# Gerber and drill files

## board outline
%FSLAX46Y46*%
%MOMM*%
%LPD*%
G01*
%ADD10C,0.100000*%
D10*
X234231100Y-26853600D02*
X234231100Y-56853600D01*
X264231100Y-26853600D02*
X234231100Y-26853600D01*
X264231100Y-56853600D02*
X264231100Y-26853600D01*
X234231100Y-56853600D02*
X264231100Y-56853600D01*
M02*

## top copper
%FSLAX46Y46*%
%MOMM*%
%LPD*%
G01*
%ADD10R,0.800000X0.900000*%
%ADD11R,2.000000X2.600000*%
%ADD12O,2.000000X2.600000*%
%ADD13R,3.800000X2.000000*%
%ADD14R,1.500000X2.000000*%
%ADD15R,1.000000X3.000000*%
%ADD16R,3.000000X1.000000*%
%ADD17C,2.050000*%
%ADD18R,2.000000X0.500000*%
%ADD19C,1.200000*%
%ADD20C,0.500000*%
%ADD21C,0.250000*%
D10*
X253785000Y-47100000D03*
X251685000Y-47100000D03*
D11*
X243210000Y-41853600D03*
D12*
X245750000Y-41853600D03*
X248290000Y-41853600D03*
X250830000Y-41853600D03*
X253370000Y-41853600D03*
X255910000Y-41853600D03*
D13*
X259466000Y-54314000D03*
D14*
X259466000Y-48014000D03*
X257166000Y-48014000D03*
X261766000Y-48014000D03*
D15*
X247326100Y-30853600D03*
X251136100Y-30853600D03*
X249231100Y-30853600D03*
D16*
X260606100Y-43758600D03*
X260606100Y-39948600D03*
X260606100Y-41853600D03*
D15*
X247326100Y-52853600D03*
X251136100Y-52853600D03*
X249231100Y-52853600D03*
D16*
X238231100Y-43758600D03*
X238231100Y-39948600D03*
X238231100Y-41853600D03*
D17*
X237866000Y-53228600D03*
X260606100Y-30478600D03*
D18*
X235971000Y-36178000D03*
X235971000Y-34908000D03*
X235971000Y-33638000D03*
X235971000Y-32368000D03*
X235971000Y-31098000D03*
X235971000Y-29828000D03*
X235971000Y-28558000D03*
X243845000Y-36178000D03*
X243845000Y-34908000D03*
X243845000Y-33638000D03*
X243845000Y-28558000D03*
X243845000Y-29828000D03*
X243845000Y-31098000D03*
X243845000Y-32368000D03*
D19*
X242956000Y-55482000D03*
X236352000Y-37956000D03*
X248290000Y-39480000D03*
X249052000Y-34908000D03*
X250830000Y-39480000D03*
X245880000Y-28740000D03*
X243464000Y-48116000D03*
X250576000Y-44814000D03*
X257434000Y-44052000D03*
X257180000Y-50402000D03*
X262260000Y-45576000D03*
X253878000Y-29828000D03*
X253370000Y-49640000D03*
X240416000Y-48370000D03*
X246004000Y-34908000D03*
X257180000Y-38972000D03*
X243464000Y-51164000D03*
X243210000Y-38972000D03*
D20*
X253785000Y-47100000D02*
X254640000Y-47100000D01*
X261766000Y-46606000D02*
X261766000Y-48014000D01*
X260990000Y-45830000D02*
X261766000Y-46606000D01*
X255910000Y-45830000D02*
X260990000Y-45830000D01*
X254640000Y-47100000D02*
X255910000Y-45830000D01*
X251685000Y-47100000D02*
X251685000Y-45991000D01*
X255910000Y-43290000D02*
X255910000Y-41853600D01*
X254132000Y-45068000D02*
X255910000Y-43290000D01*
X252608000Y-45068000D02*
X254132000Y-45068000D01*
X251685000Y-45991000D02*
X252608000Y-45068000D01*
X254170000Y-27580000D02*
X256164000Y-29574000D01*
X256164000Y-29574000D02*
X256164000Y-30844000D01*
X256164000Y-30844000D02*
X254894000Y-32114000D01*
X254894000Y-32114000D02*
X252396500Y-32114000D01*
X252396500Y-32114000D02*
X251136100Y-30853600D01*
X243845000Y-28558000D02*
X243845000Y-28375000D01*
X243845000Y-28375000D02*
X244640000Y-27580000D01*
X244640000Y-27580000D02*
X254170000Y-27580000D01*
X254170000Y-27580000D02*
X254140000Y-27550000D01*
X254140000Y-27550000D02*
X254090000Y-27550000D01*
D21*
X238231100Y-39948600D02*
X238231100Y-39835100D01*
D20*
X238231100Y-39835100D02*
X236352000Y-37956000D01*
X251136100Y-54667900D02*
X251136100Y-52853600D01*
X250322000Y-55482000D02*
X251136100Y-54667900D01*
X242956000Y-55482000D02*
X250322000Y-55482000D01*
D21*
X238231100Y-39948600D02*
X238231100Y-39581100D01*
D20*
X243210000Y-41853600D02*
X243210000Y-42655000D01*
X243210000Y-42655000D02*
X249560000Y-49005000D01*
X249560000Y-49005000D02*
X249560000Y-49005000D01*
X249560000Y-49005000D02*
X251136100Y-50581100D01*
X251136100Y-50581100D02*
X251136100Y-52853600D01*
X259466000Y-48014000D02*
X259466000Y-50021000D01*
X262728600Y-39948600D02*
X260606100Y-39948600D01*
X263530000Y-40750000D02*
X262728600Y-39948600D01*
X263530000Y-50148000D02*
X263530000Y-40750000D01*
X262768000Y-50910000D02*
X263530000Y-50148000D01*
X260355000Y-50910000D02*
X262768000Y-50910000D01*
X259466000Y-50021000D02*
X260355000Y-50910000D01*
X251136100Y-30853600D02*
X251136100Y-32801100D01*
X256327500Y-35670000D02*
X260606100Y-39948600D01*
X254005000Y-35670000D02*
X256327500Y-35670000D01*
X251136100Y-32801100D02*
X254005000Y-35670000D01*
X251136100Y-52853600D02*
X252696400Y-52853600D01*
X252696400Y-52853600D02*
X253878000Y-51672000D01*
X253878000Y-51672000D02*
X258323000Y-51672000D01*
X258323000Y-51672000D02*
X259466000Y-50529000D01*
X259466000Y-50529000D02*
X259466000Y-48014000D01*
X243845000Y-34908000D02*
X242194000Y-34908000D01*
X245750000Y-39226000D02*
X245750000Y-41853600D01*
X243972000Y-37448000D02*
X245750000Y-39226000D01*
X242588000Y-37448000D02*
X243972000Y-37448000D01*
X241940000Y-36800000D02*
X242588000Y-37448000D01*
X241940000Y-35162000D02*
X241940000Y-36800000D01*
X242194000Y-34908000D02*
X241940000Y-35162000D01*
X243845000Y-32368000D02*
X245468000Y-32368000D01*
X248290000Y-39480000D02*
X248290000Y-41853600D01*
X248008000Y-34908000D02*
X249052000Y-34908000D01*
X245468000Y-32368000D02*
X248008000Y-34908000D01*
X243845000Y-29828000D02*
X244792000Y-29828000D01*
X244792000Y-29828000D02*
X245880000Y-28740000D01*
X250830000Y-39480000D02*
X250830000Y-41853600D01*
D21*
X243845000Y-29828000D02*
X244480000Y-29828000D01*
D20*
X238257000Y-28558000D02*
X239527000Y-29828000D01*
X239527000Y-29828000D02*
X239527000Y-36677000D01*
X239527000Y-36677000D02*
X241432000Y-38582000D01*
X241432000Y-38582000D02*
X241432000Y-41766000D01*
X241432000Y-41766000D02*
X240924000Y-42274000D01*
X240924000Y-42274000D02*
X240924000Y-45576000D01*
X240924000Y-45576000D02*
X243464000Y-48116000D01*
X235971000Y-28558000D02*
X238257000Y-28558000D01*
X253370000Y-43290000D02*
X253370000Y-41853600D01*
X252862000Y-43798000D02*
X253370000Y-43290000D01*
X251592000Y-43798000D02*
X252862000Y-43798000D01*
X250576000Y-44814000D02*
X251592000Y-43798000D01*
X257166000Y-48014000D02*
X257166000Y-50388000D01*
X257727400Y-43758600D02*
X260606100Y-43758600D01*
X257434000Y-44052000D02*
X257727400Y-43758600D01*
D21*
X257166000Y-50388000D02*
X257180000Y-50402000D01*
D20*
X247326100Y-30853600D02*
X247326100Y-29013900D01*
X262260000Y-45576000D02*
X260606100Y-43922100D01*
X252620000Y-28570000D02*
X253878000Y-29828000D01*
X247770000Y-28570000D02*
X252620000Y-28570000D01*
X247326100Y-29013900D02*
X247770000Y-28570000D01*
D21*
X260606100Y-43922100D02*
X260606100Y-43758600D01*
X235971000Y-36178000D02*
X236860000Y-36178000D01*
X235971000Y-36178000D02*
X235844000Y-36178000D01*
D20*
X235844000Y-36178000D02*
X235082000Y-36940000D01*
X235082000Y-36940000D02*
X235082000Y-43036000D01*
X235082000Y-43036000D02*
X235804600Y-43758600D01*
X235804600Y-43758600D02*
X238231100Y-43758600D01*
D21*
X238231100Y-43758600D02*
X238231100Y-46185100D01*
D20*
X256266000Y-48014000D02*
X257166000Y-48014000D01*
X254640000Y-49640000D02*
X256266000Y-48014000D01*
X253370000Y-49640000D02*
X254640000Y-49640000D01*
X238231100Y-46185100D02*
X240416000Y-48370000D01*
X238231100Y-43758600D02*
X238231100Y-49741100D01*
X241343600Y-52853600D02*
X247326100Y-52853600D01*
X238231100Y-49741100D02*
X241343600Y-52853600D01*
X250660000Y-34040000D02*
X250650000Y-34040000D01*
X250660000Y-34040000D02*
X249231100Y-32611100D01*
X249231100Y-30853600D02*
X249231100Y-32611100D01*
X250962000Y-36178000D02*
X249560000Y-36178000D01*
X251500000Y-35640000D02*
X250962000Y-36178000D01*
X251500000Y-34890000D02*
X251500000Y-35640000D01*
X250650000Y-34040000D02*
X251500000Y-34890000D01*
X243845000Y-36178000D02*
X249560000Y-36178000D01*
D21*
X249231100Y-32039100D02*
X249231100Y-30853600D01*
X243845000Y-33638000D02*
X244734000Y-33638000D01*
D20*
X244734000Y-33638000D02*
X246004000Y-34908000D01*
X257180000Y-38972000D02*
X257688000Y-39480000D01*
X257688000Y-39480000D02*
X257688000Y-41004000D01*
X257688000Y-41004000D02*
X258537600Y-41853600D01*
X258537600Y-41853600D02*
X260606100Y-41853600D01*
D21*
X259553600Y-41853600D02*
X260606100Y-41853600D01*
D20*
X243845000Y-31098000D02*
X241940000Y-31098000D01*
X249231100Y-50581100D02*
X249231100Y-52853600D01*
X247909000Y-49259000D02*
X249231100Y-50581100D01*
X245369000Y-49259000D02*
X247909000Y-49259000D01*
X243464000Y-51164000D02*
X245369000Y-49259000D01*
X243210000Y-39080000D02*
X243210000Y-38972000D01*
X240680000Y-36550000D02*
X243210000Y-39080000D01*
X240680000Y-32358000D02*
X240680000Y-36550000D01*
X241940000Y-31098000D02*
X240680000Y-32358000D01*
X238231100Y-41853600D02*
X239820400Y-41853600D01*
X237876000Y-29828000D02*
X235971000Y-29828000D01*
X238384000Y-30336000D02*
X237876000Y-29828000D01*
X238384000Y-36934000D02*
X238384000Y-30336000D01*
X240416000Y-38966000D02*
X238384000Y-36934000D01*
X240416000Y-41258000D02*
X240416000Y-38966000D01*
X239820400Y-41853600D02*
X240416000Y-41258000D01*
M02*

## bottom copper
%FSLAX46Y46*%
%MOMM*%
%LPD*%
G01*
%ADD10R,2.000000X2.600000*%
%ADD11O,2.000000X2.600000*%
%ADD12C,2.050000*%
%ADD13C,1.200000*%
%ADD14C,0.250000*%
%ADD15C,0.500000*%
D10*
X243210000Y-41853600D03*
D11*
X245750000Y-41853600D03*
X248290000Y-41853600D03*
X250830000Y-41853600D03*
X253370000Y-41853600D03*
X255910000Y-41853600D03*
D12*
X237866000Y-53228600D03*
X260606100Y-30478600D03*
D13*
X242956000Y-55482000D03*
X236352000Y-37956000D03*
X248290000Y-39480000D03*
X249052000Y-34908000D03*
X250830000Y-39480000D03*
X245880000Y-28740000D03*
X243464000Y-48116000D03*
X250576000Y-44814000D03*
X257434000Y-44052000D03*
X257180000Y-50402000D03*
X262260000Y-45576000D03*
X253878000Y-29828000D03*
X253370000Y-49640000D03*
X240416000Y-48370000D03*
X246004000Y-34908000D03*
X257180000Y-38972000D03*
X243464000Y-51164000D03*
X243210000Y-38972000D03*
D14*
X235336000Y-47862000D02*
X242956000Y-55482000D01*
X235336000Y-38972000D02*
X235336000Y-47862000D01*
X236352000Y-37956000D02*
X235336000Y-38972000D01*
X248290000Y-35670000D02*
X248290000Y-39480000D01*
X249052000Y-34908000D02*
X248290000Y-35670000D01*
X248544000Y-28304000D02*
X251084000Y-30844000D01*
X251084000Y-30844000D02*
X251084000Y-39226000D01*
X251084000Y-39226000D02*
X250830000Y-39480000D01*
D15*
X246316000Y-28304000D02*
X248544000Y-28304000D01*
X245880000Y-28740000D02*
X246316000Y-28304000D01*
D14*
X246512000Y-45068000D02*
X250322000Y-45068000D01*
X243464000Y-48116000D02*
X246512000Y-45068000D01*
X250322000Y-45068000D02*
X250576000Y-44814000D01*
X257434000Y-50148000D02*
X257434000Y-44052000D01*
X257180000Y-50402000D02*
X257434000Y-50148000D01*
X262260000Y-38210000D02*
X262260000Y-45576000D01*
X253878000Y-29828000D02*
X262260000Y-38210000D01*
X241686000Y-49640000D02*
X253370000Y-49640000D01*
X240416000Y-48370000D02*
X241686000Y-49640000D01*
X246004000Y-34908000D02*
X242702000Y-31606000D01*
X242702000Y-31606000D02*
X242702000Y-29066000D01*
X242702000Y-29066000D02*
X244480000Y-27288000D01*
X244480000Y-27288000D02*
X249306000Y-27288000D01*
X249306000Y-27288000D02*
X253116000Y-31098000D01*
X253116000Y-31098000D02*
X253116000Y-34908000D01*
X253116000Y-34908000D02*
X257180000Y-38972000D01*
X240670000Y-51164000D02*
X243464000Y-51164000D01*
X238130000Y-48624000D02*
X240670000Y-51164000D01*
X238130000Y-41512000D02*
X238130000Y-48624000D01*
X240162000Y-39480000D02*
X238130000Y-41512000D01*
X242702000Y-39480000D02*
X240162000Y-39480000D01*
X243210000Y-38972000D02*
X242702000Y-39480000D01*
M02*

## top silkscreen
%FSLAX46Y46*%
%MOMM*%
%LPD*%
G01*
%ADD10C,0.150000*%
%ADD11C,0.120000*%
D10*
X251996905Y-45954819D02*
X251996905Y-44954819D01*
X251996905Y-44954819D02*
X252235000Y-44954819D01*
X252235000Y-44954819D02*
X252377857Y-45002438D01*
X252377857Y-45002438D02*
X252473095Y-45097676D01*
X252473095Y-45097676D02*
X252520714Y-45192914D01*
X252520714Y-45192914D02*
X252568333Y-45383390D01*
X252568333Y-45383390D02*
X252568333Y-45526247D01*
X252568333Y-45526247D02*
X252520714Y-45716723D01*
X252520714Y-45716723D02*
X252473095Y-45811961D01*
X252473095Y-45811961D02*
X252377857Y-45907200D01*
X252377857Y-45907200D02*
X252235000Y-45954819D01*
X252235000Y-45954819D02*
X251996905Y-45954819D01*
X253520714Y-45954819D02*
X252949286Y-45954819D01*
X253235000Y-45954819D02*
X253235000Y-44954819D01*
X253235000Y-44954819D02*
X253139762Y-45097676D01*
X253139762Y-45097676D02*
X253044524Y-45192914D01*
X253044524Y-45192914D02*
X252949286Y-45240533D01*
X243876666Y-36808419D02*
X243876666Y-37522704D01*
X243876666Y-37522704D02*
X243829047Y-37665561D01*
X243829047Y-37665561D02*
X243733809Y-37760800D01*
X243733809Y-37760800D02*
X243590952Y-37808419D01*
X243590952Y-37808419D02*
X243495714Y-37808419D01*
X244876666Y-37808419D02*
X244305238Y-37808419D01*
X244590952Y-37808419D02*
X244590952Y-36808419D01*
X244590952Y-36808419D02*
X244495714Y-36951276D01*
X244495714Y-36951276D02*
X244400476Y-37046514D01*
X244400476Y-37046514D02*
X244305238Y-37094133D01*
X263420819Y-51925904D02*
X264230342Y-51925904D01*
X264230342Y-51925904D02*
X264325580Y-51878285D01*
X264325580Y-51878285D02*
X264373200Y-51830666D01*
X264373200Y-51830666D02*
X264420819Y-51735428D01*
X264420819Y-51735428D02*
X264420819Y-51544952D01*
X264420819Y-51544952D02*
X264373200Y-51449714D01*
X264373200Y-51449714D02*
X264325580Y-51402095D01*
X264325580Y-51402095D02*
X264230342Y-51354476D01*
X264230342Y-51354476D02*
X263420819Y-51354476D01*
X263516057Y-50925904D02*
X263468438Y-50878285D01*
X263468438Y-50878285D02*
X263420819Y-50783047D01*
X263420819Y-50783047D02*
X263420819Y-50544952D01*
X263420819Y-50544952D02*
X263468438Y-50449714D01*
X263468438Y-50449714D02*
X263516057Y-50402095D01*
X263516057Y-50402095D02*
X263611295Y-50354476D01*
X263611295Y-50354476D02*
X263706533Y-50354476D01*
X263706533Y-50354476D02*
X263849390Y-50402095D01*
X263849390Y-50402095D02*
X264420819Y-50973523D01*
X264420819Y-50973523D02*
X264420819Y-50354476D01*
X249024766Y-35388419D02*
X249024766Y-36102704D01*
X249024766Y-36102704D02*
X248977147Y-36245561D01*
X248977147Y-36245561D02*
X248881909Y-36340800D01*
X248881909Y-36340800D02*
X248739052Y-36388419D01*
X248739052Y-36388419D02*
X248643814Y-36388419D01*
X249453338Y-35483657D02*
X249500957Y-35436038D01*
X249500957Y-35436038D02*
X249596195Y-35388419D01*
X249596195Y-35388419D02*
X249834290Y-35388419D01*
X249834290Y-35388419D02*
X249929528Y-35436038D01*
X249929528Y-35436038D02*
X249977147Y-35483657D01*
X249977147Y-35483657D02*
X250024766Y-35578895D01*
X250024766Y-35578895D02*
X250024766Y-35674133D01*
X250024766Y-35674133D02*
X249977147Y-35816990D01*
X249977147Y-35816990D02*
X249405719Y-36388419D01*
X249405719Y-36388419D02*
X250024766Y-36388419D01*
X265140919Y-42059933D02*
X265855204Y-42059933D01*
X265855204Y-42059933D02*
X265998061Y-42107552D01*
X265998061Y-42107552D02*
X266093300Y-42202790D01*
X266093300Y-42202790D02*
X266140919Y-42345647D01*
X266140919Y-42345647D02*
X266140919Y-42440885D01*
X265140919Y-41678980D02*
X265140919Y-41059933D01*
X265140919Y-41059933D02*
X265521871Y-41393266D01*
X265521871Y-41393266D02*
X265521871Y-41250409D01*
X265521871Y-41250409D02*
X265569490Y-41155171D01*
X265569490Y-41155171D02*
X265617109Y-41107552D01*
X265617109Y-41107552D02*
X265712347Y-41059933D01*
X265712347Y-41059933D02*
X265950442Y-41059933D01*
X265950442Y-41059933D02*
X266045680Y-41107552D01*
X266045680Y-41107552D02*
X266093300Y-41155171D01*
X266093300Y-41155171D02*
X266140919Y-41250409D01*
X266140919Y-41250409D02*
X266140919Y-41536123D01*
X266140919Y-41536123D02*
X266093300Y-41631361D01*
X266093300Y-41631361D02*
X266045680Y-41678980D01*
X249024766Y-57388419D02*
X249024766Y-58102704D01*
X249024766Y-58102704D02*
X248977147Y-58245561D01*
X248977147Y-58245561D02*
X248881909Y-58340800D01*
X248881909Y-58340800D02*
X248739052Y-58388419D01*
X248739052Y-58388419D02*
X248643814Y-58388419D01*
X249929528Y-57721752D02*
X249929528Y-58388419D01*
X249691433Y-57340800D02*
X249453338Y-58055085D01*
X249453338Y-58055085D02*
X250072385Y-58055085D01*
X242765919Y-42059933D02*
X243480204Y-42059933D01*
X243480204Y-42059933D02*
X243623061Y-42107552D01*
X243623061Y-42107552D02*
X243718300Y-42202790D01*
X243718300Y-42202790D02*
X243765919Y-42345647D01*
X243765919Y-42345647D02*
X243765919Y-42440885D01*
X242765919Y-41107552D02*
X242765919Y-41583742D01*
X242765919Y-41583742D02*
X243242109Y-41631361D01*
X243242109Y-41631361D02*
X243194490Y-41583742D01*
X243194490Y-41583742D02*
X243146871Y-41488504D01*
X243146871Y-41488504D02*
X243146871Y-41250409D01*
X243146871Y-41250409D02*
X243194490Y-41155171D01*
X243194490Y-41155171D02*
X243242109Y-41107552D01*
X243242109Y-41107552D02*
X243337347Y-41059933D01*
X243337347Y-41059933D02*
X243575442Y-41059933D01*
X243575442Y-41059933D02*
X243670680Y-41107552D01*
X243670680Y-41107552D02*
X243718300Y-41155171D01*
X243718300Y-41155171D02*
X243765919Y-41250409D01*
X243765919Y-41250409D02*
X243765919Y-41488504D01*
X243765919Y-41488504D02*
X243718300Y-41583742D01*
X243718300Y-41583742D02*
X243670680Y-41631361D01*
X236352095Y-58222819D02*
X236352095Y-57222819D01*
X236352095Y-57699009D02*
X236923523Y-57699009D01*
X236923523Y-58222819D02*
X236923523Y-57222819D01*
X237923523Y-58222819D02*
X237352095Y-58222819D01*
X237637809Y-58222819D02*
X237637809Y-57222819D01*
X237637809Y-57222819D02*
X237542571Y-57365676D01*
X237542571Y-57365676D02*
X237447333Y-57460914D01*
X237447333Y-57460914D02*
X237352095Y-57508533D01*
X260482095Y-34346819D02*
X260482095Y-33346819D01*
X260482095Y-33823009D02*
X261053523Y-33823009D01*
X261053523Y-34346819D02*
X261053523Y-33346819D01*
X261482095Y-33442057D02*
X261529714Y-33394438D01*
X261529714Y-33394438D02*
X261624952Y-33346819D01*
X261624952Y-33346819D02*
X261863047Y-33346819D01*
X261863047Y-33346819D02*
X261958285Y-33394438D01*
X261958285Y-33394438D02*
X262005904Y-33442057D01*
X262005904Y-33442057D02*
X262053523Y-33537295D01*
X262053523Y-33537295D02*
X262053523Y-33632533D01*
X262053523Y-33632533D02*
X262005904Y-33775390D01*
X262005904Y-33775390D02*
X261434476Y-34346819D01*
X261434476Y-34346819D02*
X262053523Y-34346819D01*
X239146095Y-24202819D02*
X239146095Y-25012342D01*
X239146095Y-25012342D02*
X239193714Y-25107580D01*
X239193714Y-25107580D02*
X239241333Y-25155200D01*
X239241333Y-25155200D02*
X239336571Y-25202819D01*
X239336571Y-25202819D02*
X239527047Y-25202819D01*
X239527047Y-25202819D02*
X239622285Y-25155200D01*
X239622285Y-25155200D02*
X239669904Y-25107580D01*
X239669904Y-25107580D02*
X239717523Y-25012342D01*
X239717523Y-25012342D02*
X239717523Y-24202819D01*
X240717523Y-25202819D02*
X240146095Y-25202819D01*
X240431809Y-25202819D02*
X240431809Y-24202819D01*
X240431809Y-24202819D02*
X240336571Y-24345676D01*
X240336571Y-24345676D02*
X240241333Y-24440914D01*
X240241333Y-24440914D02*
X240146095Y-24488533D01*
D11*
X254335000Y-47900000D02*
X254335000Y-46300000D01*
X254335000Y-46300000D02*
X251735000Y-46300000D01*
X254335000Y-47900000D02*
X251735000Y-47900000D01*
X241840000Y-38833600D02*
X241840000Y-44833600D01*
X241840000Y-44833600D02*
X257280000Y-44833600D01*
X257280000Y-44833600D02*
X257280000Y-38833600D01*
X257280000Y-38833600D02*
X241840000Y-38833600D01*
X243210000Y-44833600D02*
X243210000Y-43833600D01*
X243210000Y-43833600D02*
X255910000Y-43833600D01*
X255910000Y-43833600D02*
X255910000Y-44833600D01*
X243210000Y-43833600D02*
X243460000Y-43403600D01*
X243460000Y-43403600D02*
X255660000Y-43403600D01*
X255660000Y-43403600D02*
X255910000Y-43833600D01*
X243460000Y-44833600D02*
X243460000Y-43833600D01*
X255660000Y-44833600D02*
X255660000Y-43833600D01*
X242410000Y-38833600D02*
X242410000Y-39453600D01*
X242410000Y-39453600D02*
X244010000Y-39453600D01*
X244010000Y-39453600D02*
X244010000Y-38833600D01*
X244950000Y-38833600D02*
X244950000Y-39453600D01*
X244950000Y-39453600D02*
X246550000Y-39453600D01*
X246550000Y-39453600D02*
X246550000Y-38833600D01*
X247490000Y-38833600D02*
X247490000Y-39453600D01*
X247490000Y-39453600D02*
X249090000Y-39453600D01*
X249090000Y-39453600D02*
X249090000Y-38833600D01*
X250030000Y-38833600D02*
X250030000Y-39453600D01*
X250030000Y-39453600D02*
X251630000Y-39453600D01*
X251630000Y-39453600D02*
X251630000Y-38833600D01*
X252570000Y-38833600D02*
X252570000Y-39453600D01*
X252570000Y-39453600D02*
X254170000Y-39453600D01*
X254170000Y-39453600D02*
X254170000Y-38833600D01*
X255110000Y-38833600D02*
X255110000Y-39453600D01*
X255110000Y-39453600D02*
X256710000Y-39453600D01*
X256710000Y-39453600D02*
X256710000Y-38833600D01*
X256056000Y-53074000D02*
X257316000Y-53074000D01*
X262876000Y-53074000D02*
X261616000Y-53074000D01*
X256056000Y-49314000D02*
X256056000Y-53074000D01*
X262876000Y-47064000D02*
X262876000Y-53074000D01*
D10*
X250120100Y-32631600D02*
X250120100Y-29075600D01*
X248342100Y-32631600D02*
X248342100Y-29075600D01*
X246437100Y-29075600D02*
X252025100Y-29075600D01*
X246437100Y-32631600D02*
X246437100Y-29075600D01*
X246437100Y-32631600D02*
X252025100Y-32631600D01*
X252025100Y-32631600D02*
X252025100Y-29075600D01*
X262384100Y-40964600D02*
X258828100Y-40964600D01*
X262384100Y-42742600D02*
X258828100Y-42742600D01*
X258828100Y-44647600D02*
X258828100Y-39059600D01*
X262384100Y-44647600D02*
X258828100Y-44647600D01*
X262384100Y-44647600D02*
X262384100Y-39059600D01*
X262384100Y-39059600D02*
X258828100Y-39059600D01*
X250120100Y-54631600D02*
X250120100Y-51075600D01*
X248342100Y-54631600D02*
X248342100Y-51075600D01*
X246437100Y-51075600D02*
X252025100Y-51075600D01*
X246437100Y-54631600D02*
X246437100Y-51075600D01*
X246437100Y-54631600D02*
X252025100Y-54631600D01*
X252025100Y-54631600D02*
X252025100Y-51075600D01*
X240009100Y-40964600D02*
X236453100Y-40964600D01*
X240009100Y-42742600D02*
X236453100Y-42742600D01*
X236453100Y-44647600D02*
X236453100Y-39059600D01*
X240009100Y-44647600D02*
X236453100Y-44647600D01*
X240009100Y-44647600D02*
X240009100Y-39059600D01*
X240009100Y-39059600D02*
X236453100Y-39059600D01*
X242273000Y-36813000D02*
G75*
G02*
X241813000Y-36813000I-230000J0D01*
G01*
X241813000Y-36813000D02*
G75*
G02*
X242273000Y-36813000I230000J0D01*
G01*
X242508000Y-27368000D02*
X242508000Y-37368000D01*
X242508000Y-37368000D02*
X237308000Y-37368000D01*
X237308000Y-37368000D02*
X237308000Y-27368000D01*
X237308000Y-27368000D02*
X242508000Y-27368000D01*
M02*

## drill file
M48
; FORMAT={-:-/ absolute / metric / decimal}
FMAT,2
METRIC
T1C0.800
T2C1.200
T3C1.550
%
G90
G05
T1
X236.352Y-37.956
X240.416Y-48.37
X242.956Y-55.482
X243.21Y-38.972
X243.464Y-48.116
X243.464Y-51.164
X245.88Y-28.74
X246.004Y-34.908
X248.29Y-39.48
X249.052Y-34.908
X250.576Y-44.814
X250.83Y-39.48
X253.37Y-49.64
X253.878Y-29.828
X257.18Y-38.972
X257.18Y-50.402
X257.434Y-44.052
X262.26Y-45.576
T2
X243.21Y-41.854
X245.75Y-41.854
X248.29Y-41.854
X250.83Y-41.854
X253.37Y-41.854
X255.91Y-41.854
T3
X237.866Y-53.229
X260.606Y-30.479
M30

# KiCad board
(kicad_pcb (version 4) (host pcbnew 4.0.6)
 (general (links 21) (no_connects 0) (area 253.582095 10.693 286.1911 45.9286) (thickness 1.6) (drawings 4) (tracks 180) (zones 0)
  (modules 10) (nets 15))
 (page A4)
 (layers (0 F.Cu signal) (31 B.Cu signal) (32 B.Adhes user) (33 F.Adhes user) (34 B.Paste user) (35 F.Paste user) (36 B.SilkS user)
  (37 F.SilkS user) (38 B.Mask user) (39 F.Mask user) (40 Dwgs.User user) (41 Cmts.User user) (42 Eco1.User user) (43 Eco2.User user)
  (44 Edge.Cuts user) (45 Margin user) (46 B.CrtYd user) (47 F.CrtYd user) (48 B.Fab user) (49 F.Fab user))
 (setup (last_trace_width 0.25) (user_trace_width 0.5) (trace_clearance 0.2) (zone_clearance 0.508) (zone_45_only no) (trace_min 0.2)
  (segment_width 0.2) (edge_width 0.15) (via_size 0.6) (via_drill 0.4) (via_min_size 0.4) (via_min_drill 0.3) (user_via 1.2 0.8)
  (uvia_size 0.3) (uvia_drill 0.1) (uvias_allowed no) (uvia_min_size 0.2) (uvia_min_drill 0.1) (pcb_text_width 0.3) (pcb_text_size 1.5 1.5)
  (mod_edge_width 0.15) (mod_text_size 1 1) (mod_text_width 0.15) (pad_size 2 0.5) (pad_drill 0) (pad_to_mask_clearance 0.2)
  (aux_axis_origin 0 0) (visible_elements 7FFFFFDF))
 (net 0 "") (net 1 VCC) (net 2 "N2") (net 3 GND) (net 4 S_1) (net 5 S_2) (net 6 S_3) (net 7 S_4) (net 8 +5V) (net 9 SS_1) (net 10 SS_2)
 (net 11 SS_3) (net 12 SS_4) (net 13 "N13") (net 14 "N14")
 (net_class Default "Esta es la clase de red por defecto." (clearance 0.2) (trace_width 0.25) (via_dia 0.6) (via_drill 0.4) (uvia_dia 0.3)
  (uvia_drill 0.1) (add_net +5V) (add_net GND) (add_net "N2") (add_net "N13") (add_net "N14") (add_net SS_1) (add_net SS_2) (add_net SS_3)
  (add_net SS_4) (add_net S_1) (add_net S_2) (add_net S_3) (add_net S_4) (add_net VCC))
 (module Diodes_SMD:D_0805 (layer F.Cu) (at 252.735 47.1 180)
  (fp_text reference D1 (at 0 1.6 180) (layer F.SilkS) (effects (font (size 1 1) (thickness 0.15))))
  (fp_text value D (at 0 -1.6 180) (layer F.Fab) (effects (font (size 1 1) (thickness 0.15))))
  (fp_line (start -1.6 -0.8) (end -1.6 0.8) (layer F.SilkS) (width 0.12))
  (fp_line (start -1.6 0.8) (end 1 0.8) (layer F.SilkS) (width 0.12))
  (fp_line (start -1.6 -0.8) (end 1 -0.8) (layer F.SilkS) (width 0.12))
  (pad 1 smd rect (at -1.05 0 180) (size 0.8 0.9) (layers F.Cu F.Paste F.Mask) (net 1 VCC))
  (pad 2 smd rect (at 1.05 0 180) (size 0.8 0.9) (layers F.Cu F.Paste F.Mask) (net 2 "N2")))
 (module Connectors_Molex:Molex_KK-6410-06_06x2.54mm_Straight (layer F.Cu) (at 243.21 41.8536)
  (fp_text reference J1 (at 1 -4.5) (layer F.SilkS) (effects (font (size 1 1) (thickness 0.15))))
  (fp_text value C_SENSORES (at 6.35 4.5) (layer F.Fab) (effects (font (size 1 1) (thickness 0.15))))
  (fp_line (start -1.37 -3.02) (end -1.37 2.98) (layer F.SilkS) (width 0.12))
  (fp_line (start -1.37 2.98) (end 14.07 2.98) (layer F.SilkS) (width 0.12))
  (fp_line (start 14.07 2.98) (end 14.07 -3.02) (layer F.SilkS) (width 0.12))
  (fp_line (start 14.07 -3.02) (end -1.37 -3.02) (layer F.SilkS) (width 0.12))
  (fp_line (start 0 2.98) (end 0 1.98) (layer F.SilkS) (width 0.12))
  (fp_line (start 0 1.98) (end 12.7 1.98) (layer F.SilkS) (width 0.12))
  (fp_line (start 12.7 1.98) (end 12.7 2.98) (layer F.SilkS) (width 0.12))
  (fp_line (start 0 1.98) (end 0.25 1.55) (layer F.SilkS) (width 0.12))
  (fp_line (start 0.25 1.55) (end 12.45 1.55) (layer F.SilkS) (width 0.12))
  (fp_line (start 12.45 1.55) (end 12.7 1.98) (layer F.SilkS) (width 0.12))
  (fp_line (start 0.25 2.98) (end 0.25 1.98) (layer F.SilkS) (width 0.12))
  (fp_line (start 12.45 2.98) (end 12.45 1.98) (layer F.SilkS) (width 0.12))
  (fp_line (start -0.8 -3.02) (end -0.8 -2.4) (layer F.SilkS) (width 0.12))
  (fp_line (start -0.8 -2.4) (end 0.8 -2.4) (layer F.SilkS) (width 0.12))
  (fp_line (start 0.8 -2.4) (end 0.8 -3.02) (layer F.SilkS) (width 0.12))
  (fp_line (start 1.74 -3.02) (end 1.74 -2.4) (layer F.SilkS) (width 0.12))
  (fp_line (start 1.74 -2.4) (end 3.34 -2.4) (layer F.SilkS) (width 0.12))
  (fp_line (start 3.34 -2.4) (end 3.34 -3.02) (layer F.SilkS) (width 0.12))
  (fp_line (start 4.28 -3.02) (end 4.28 -2.4) (layer F.SilkS) (width 0.12))
  (fp_line (start 4.28 -2.4) (end 5.88 -2.4) (layer F.SilkS) (width 0.12))
  (fp_line (start 5.88 -2.4) (end 5.88 -3.02) (layer F.SilkS) (width 0.12))
  (fp_line (start 6.82 -3.02) (end 6.82 -2.4) (layer F.SilkS) (width 0.12))
  (fp_line (start 6.82 -2.4) (end 8.42 -2.4) (layer F.SilkS) (width 0.12))
  (fp_line (start 8.42 -2.4) (end 8.42 -3.02) (layer F.SilkS) (width 0.12))
  (fp_line (start 9.36 -3.02) (end 9.36 -2.4) (layer F.SilkS) (width 0.12))
  (fp_line (start 9.36 -2.4) (end 10.96 -2.4) (layer F.SilkS) (width 0.12))
  (fp_line (start 10.96 -2.4) (end 10.96 -3.02) (layer F.SilkS) (width 0.12))
  (fp_line (start 11.9 -3.02) (end 11.9 -2.4) (layer F.SilkS) (width 0.12))
  (fp_line (start 11.9 -2.4) (end 13.5 -2.4) (layer F.SilkS) (width 0.12))
  (fp_line (start 13.5 -2.4) (end 13.5 -3.02) (layer F.SilkS) (width 0.12))
  (pad 1 thru_hole rect (at 0 0) (size 2 2.6) (drill 1.2) (layers *.Cu *.Mask) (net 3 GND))
  (pad 2 thru_hole oval (at 2.54 0) (size 2 2.6) (drill 1.2) (layers *.Cu *.Mask) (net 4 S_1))
  (pad 3 thru_hole oval (at 5.08 0) (size 2 2.6) (drill 1.2) (layers *.Cu *.Mask) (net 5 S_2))
  (pad 4 thru_hole oval (at 7.62 0) (size 2 2.6) (drill 1.2) (layers *.Cu *.Mask) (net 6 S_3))
  (pad 5 thru_hole oval (at 10.16 0) (size 2 2.6) (drill 1.2) (layers *.Cu *.Mask) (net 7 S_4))
  (pad 6 thru_hole oval (at 12.7 0) (size 2 2.6) (drill 1.2) (layers *.Cu *.Mask) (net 2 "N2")))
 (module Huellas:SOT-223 (layer F.Cu) (at 259.466 51.164 270)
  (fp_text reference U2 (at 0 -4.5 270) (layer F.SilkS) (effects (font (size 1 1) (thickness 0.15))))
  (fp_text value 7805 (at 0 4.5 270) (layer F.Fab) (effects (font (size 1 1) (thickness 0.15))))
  (fp_line (start 1.91 3.41) (end 1.91 2.15) (layer F.SilkS) (width 0.12))
  (fp_line (start 1.91 -3.41) (end 1.91 -2.15) (layer F.SilkS) (width 0.12))
  (fp_line (start -1.85 3.41) (end 1.91 3.41) (layer F.SilkS) (width 0.12))
  (fp_line (start -4.1 -3.41) (end 1.91 -3.41) (layer F.SilkS) (width 0.12))
  (pad "" smd rect (at 3.15 0 270) (size 2 3.8) (layers F.Cu F.Paste F.Mask))
  (pad GND smd rect (at -3.15 0 270) (size 2 1.5) (layers F.Cu F.Paste F.Mask) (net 3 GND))
  (pad VO smd rect (at -3.15 2.3 270) (size 2 1.5) (layers F.Cu F.Paste F.Mask) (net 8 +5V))
  (pad VI smd rect (at -3.15 -2.3 270) (size 2 1.5) (layers F.Cu F.Paste F.Mask) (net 1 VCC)))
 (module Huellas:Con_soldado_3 (layer F.Cu) (at 249.2311 30.8536)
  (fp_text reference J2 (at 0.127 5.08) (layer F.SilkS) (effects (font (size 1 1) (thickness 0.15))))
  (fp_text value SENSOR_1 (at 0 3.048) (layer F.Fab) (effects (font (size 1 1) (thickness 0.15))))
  (fp_line (start 0.889 1.778) (end 0.889 -1.778) (layer F.SilkS) (width 0.15))
  (fp_line (start -0.889 1.778) (end -0.889 -1.778) (layer F.SilkS) (width 0.15))
  (fp_line (start -2.794 -1.778) (end 2.794 -1.778) (layer F.SilkS) (width 0.15))
  (fp_line (start -2.794 1.778) (end -2.794 -1.778) (layer F.SilkS) (width 0.15))
  (fp_line (start -2.794 1.778) (end 2.794 1.778) (layer F.SilkS) (width 0.15))
  (fp_line (start 2.794 1.778) (end 2.794 -1.778) (layer F.SilkS) (width 0.15))
  (pad 1 smd rect (at -1.905 0) (size 1 3) (layers F.Cu F.Paste F.Mask) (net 8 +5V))
  (pad 3 smd rect (at 1.905 0) (size 1 3) (layers F.Cu F.Paste F.Mask) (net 3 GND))
  (pad 2 smd rect (at 0 0) (size 1 3) (layers F.Cu F.Paste F.Mask) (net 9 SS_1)))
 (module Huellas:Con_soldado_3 (layer F.Cu) (at 260.6061 41.8536 90)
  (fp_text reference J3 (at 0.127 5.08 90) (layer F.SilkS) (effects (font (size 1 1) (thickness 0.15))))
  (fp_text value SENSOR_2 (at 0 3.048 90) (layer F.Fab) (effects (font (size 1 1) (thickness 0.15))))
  (fp_line (start 0.889 1.778) (end 0.889 -1.778) (layer F.SilkS) (width 0.15))
  (fp_line (start -0.889 1.778) (end -0.889 -1.778) (layer F.SilkS) (width 0.15))
  (fp_line (start -2.794 -1.778) (end 2.794 -1.778) (layer F.SilkS) (width 0.15))
  (fp_line (start -2.794 1.778) (end -2.794 -1.778) (layer F.SilkS) (width 0.15))
  (fp_line (start -2.794 1.778) (end 2.794 1.778) (layer F.SilkS) (width 0.15))
  (fp_line (start 2.794 1.778) (end 2.794 -1.778) (layer F.SilkS) (width 0.15))
  (pad 1 smd rect (at -1.905 0 90) (size 1 3) (layers F.Cu F.Paste F.Mask) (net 8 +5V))
  (pad 3 smd rect (at 1.905 0 90) (size 1 3) (layers F.Cu F.Paste F.Mask) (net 3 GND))
  (pad 2 smd rect (at 0 0 90) (size 1 3) (layers F.Cu F.Paste F.Mask) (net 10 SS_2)))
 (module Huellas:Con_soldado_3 (layer F.Cu) (at 249.2311 52.8536)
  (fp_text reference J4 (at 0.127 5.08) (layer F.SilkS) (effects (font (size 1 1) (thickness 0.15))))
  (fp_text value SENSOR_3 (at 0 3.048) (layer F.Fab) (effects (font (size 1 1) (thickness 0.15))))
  (fp_line (start 0.889 1.778) (end 0.889 -1.778) (layer F.SilkS) (width 0.15))
  (fp_line (start -0.889 1.778) (end -0.889 -1.778) (layer F.SilkS) (width 0.15))
  (fp_line (start -2.794 -1.778) (end 2.794 -1.778) (layer F.SilkS) (width 0.15))
  (fp_line (start -2.794 1.778) (end -2.794 -1.778) (layer F.SilkS) (width 0.15))
  (fp_line (start -2.794 1.778) (end 2.794 1.778) (layer F.SilkS) (width 0.15))
  (fp_line (start 2.794 1.778) (end 2.794 -1.778) (layer F.SilkS) (width 0.15))
  (pad 1 smd rect (at -1.905 0) (size 1 3) (layers F.Cu F.Paste F.Mask) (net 8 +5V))
  (pad 3 smd rect (at 1.905 0) (size 1 3) (layers F.Cu F.Paste F.Mask) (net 3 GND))
  (pad 2 smd rect (at 0 0) (size 1 3) (layers F.Cu F.Paste F.Mask) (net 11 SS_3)))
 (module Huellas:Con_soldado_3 (layer F.Cu) (at 238.2311 41.8536 90)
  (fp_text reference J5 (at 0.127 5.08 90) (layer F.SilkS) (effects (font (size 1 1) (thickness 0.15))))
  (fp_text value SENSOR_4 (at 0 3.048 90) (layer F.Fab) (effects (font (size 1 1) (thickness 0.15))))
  (fp_line (start 0.889 1.778) (end 0.889 -1.778) (layer F.SilkS) (width 0.15))
  (fp_line (start -0.889 1.778) (end -0.889 -1.778) (layer F.SilkS) (width 0.15))
  (fp_line (start -2.794 -1.778) (end 2.794 -1.778) (layer F.SilkS) (width 0.15))
  (fp_line (start -2.794 1.778) (end -2.794 -1.778) (layer F.SilkS) (width 0.15))
  (fp_line (start -2.794 1.778) (end 2.794 1.778) (layer F.SilkS) (width 0.15))
  (fp_line (start 2.794 1.778) (end 2.794 -1.778) (layer F.SilkS) (width 0.15))
  (pad 1 smd rect (at -1.905 0 90) (size 1 3) (layers F.Cu F.Paste F.Mask) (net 8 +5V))
  (pad 3 smd rect (at 1.905 0 90) (size 1 3) (layers F.Cu F.Paste F.Mask) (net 3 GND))
  (pad 2 smd rect (at 0 0 90) (size 1 3) (layers F.Cu F.Paste F.Mask) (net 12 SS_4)))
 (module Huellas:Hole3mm (layer F.Cu) (at 237.114 53.958)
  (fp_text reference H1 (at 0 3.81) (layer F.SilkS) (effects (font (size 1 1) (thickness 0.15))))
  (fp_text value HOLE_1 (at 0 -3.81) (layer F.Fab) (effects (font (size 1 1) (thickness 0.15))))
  (pad 1 thru_hole circle (at 0.752 -0.7294) (size 2.05 2.05) (drill 1.55) (layers *.Cu *.Mask) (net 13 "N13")))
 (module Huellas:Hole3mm (layer F.Cu) (at 261.244 30.082)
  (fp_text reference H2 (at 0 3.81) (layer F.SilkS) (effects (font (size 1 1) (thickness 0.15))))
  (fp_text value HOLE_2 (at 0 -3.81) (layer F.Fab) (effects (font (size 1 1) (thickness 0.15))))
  (pad 1 thru_hole circle (at -0.6379 0.3966) (size 2.05 2.05) (drill 1.55) (layers *.Cu *.Mask) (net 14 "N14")))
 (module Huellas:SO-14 (layer F.Cu) (at 239.908 32.368 180)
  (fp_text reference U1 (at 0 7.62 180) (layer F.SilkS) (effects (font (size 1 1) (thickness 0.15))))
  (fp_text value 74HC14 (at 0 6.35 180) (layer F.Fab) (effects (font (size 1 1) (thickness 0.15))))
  (fp_circle (center -2.135 -4.445) (end -1.905 -4.445) (layer F.SilkS) (width 0.15))
  (fp_line (start -2.6 5) (end -2.6 -5) (layer F.SilkS) (width 0.15))
  (fp_line (start -2.6 -5) (end 2.6 -5) (layer F.SilkS) (width 0.15))
  (fp_line (start 2.6 -5) (end 2.6 5) (layer F.SilkS) (width 0.15))
  (fp_line (start 2.6 5) (end -2.6 5) (layer F.SilkS) (width 0.15))
  (pad +5V smd rect (at 3.937 -3.81 180) (size 2 0.5) (layers F.Cu F.Paste F.Mask) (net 8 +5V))
  (pad 13 smd rect (at 3.937 -2.54 180) (size 2 0.5) (layers F.Cu F.Paste F.Mask))
  (pad 12 smd rect (at 3.937 -1.27 180) (size 2 0.5) (layers F.Cu F.Paste F.Mask))
  (pad 11 smd rect (at 3.937 0 180) (size 2 0.5) (layers F.Cu F.Paste F.Mask))
  (pad 10 smd rect (at 3.937 1.27 180) (size 2 0.5) (layers F.Cu F.Paste F.Mask))
  (pad 9 smd rect (at 3.937 2.54 180) (size 2 0.5) (layers F.Cu F.Paste F.Mask) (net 12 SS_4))
  (pad 8 smd rect (at 3.937 3.81 180) (size 2 0.5) (layers F.Cu F.Paste F.Mask) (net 7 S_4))
  (pad 1 smd rect (at -3.937 -3.81 180) (size 2 0.5) (layers F.Cu F.Paste F.Mask) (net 9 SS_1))
  (pad 2 smd rect (at -3.937 -2.54 180) (size 2 0.5) (layers F.Cu F.Paste F.Mask) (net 4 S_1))
  (pad 3 smd rect (at -3.937 -1.27 180) (size 2 0.5) (layers F.Cu F.Paste F.Mask) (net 10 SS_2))
  (pad GND smd rect (at -3.937 3.81 180) (size 2 0.5) (layers F.Cu F.Paste F.Mask) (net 3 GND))
  (pad 6 smd rect (at -3.937 2.54 180) (size 2 0.5) (layers F.Cu F.Paste F.Mask) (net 6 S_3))
  (pad 5 smd rect (at -3.937 1.27 180) (size 2 0.5) (layers F.Cu F.Paste F.Mask) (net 11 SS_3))
  (pad 4 smd rect (at -3.937 0 180) (size 2 0.5) (layers F.Cu F.Paste F.Mask) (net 5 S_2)))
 (gr_line (start 234.2311 26.8536) (end 234.2311 56.8536) (layer Edge.Cuts) (width 0.1))
 (gr_line (start 264.2311 26.8536) (end 234.2311 26.8536) (layer Edge.Cuts) (width 0.1))
 (gr_line (start 264.2311 56.8536) (end 264.2311 26.8536) (layer Edge.Cuts) (width 0.1))
 (gr_line (start 234.2311 56.8536) (end 264.2311 56.8536) (layer Edge.Cuts) (width 0.1))
 (segment (start 253.785 47.1) (end 254.64 47.1) (width 0.5) (layer F.Cu) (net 1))
 (segment (start 261.766 46.606) (end 261.766 48.014) (width 0.5) (layer F.Cu) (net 1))
 (segment (start 260.99 45.83) (end 261.766 46.606) (width 0.5) (layer F.Cu) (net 1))
 (segment (start 255.91 45.83) (end 260.99 45.83) (width 0.5) (layer F.Cu) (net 1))
 (segment (start 254.64 47.1) (end 255.91 45.83) (width 0.5) (layer F.Cu) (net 1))
 (segment (start 251.685 47.1) (end 251.685 45.991) (width 0.5) (layer F.Cu) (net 2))
 (segment (start 255.91 43.29) (end 255.91 41.8536) (width 0.5) (layer F.Cu) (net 2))
 (segment (start 254.132 45.068) (end 255.91 43.29) (width 0.5) (layer F.Cu) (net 2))
 (segment (start 252.608 45.068) (end 254.132 45.068) (width 0.5) (layer F.Cu) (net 2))
 (segment (start 251.685 45.991) (end 252.608 45.068) (width 0.5) (layer F.Cu) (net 2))
 (segment (start 235.336 47.862) (end 242.956 55.482) (width 0.25) (layer B.Cu) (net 3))
 (segment (start 235.336 38.972) (end 235.336 47.862) (width 0.25) (layer B.Cu) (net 3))
 (segment (start 236.352 37.956) (end 235.336 38.972) (width 0.25) (layer B.Cu) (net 3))
 (segment (start 254.17 27.58) (end 256.164 29.574) (width 0.5) (layer F.Cu) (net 3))
 (segment (start 256.164 29.574) (end 256.164 30.844) (width 0.5) (layer F.Cu) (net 3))
 (segment (start 256.164 30.844) (end 254.894 32.114) (width 0.5) (layer F.Cu) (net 3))
 (segment (start 254.894 32.114) (end 252.3965 32.114) (width 0.5) (layer F.Cu) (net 3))
 (segment (start 252.3965 32.114) (end 251.1361 30.8536) (width 0.5) (layer F.Cu) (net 3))
 (segment (start 243.845 28.558) (end 243.845 28.375) (width 0.5) (layer F.Cu) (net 3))
 (segment (start 243.845 28.375) (end 244.64 27.58) (width 0.5) (layer F.Cu) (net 3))
 (segment (start 244.64 27.58) (end 254.17 27.58) (width 0.5) (layer F.Cu) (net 3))
 (segment (start 254.17 27.58) (end 254.14 27.55) (width 0.5) (layer F.Cu) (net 3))
 (segment (start 254.14 27.55) (end 254.09 27.55) (width 0.5) (layer F.Cu) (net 3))
 (segment (start 238.2311 39.9486) (end 238.2311 39.8351) (width 0.25) (layer F.Cu) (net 3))
 (segment (start 238.2311 39.8351) (end 236.352 37.956) (width 0.5) (layer F.Cu) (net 3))
 (segment (start 251.1361 54.6679) (end 251.1361 52.8536) (width 0.5) (layer F.Cu) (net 3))
 (segment (start 250.322 55.482) (end 251.1361 54.6679) (width 0.5) (layer F.Cu) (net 3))
 (segment (start 242.956 55.482) (end 250.322 55.482) (width 0.5) (layer F.Cu) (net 3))
 (via (at 242.956 55.482) (size 1.2) (drill 0.8) (layers F.Cu B.Cu) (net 3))
 (via (at 236.352 37.956) (size 1.2) (drill 0.8) (layers F.Cu B.Cu) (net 3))
 (segment (start 238.2311 39.9486) (end 238.2311 39.5811) (width 0.25) (layer F.Cu) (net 3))
 (segment (start 243.21 41.8536) (end 243.21 42.655) (width 0.5) (layer F.Cu) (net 3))
 (segment (start 243.21 42.655) (end 249.56 49.005) (width 0.5) (layer F.Cu) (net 3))
 (segment (start 249.56 49.005) (end 249.56 49.005) (width 0.5) (layer F.Cu) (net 3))
 (segment (start 249.56 49.005) (end 251.1361 50.5811) (width 0.5) (layer F.Cu) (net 3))
 (segment (start 251.1361 50.5811) (end 251.1361 52.8536) (width 0.5) (layer F.Cu) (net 3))
 (segment (start 259.466 48.014) (end 259.466 50.021) (width 0.5) (layer F.Cu) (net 3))
 (segment (start 262.7286 39.9486) (end 260.6061 39.9486) (width 0.5) (layer F.Cu) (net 3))
 (segment (start 263.53 40.75) (end 262.7286 39.9486) (width 0.5) (layer F.Cu) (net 3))
 (segment (start 263.53 50.148) (end 263.53 40.75) (width 0.5) (layer F.Cu) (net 3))
 (segment (start 262.768 50.91) (end 263.53 50.148) (width 0.5) (layer F.Cu) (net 3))
 (segment (start 260.355 50.91) (end 262.768 50.91) (width 0.5) (layer F.Cu) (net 3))
 (segment (start 259.466 50.021) (end 260.355 50.91) (width 0.5) (layer F.Cu) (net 3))
 (segment (start 251.1361 30.8536) (end 251.1361 32.8011) (width 0.5) (layer F.Cu) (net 3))
 (segment (start 256.3275 35.67) (end 260.6061 39.9486) (width 0.5) (layer F.Cu) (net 3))
 (segment (start 254.005 35.67) (end 256.3275 35.67) (width 0.5) (layer F.Cu) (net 3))
 (segment (start 251.1361 32.8011) (end 254.005 35.67) (width 0.5) (layer F.Cu) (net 3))
 (segment (start 251.1361 52.8536) (end 252.6964 52.8536) (width 0.5) (layer F.Cu) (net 3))
 (segment (start 252.6964 52.8536) (end 253.878 51.672) (width 0.5) (layer F.Cu) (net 3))
 (segment (start 253.878 51.672) (end 258.323 51.672) (width 0.5) (layer F.Cu) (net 3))
 (segment (start 258.323 51.672) (end 259.466 50.529) (width 0.5) (layer F.Cu) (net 3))
 (segment (start 259.466 50.529) (end 259.466 48.014) (width 0.5) (layer F.Cu) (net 3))
 (segment (start 243.845 34.908) (end 242.194 34.908) (width 0.5) (layer F.Cu) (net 4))
 (segment (start 245.75 39.226) (end 245.75 41.8536) (width 0.5) (layer F.Cu) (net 4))
 (segment (start 243.972 37.448) (end 245.75 39.226) (width 0.5) (layer F.Cu) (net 4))
 (segment (start 242.588 37.448) (end 243.972 37.448) (width 0.5) (layer F.Cu) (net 4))
 (segment (start 241.94 36.8) (end 242.588 37.448) (width 0.5) (layer F.Cu) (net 4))
 (segment (start 241.94 35.162) (end 241.94 36.8) (width 0.5) (layer F.Cu) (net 4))
 (segment (start 242.194 34.908) (end 241.94 35.162) (width 0.5) (layer F.Cu) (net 4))
 (segment (start 248.29 35.67) (end 248.29 39.48) (width 0.25) (layer B.Cu) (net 5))
 (segment (start 249.052 34.908) (end 248.29 35.67) (width 0.25) (layer B.Cu) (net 5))
 (segment (start 243.845 32.368) (end 245.468 32.368) (width 0.5) (layer F.Cu) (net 5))
 (segment (start 248.29 39.48) (end 248.29 41.8536) (width 0.5) (layer F.Cu) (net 5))
 (via (at 248.29 39.48) (size 1.2) (drill 0.8) (layers F.Cu B.Cu) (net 5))
 (via (at 249.052 34.908) (size 1.2) (drill 0.8) (layers F.Cu B.Cu) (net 5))
 (segment (start 248.008 34.908) (end 249.052 34.908) (width 0.5) (layer F.Cu) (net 5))
 (segment (start 245.468 32.368) (end 248.008 34.908) (width 0.5) (layer F.Cu) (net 5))
 (segment (start 248.544 28.304) (end 251.084 30.844) (width 0.25) (layer B.Cu) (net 6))
 (segment (start 251.084 30.844) (end 251.084 39.226) (width 0.25) (layer B.Cu) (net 6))
 (segment (start 251.084 39.226) (end 250.83 39.48) (width 0.25) (layer B.Cu) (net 6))
 (segment (start 246.316 28.304) (end 248.544 28.304) (width 0.5) (layer B.Cu) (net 6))
 (segment (start 245.88 28.74) (end 246.316 28.304) (width 0.5) (layer B.Cu) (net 6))
 (segment (start 243.845 29.828) (end 244.792 29.828) (width 0.5) (layer F.Cu) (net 6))
 (segment (start 244.792 29.828) (end 245.88 28.74) (width 0.5) (layer F.Cu) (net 6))
 (via (at 250.83 39.48) (size 1.2) (drill 0.8) (layers F.Cu B.Cu) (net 6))
 (segment (start 250.83 39.48) (end 250.83 41.8536) (width 0.5) (layer F.Cu) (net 6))
 (via (at 245.88 28.74) (size 1.2) (drill 0.8) (layers F.Cu B.Cu) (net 6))
 (segment (start 243.845 29.828) (end 244.48 29.828) (width 0.25) (layer F.Cu) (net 6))
 (segment (start 246.512 45.068) (end 250.322 45.068) (width 0.25) (layer B.Cu) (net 7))
 (segment (start 243.464 48.116) (end 246.512 45.068) (width 0.25) (layer B.Cu) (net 7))
 (segment (start 250.322 45.068) (end 250.576 44.814) (width 0.25) (layer B.Cu) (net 7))
 (segment (start 238.257 28.558) (end 239.527 29.828) (width 0.5) (layer F.Cu) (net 7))
 (segment (start 239.527 29.828) (end 239.527 36.677) (width 0.5) (layer F.Cu) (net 7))
 (segment (start 239.527 36.677) (end 241.432 38.582) (width 0.5) (layer F.Cu) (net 7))
 (segment (start 241.432 38.582) (end 241.432 41.766) (width 0.5) (layer F.Cu) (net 7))
 (segment (start 241.432 41.766) (end 240.924 42.274) (width 0.5) (layer F.Cu) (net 7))
 (segment (start 240.924 42.274) (end 240.924 45.576) (width 0.5) (layer F.Cu) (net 7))
 (segment (start 240.924 45.576) (end 243.464 48.116) (width 0.5) (layer F.Cu) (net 7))
 (via (at 243.464 48.116) (size 1.2) (drill 0.8) (layers F.Cu B.Cu) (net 7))
 (segment (start 235.971 28.558) (end 238.257 28.558) (width 0.5) (layer F.Cu) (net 7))
 (segment (start 253.37 43.29) (end 253.37 41.8536) (width 0.5) (layer F.Cu) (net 7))
 (segment (start 252.862 43.798) (end 253.37 43.29) (width 0.5) (layer F.Cu) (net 7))
 (segment (start 251.592 43.798) (end 252.862 43.798) (width 0.5) (layer F.Cu) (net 7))
 (segment (start 250.576 44.814) (end 251.592 43.798) (width 0.5) (layer F.Cu) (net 7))
 (via (at 250.576 44.814) (size 1.2) (drill 0.8) (layers F.Cu B.Cu) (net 7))
 (segment (start 257.434 50.148) (end 257.434 44.052) (width 0.25) (layer B.Cu) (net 8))
 (segment (start 257.18 50.402) (end 257.434 50.148) (width 0.25) (layer B.Cu) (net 8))
 (segment (start 262.26 38.21) (end 262.26 45.576) (width 0.25) (layer B.Cu) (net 8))
 (segment (start 253.878 29.828) (end 262.26 38.21) (width 0.25) (layer B.Cu) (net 8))
 (segment (start 241.686 49.64) (end 253.37 49.64) (width 0.25) (layer B.Cu) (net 8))
 (segment (start 240.416 48.37) (end 241.686 49.64) (width 0.25) (layer B.Cu) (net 8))
 (segment (start 257.166 48.014) (end 257.166 50.388) (width 0.5) (layer F.Cu) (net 8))
 (segment (start 257.7274 43.7586) (end 260.6061 43.7586) (width 0.5) (layer F.Cu) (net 8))
 (segment (start 257.434 44.052) (end 257.7274 43.7586) (width 0.5) (layer F.Cu) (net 8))
 (via (at 257.434 44.052) (size 1.2) (drill 0.8) (layers F.Cu B.Cu) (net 8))
 (via (at 257.18 50.402) (size 1.2) (drill 0.8) (layers F.Cu B.Cu) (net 8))
 (segment (start 257.166 50.388) (end 257.18 50.402) (width 0.25) (layer F.Cu) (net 8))
 (segment (start 247.3261 30.8536) (end 247.3261 29.0139) (width 0.5) (layer F.Cu) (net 8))
 (segment (start 262.26 45.576) (end 260.6061 43.9221) (width 0.5) (layer F.Cu) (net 8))
 (via (at 262.26 45.576) (size 1.2) (drill 0.8) (layers F.Cu B.Cu) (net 8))
 (via (at 253.878 29.828) (size 1.2) (drill 0.8) (layers F.Cu B.Cu) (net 8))
 (segment (start 252.62 28.57) (end 253.878 29.828) (width 0.5) (layer F.Cu) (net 8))
 (segment (start 247.77 28.57) (end 252.62 28.57) (width 0.5) (layer F.Cu) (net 8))
 (segment (start 247.3261 29.0139) (end 247.77 28.57) (width 0.5) (layer F.Cu) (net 8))
 (segment (start 260.6061 43.9221) (end 260.6061 43.7586) (width 0.25) (layer F.Cu) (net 8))
 (segment (start 235.971 36.178) (end 236.86 36.178) (width 0.25) (layer F.Cu) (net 8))
 (segment (start 235.971 36.178) (end 235.844 36.178) (width 0.25) (layer F.Cu) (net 8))
 (segment (start 235.844 36.178) (end 235.082 36.94) (width 0.5) (layer F.Cu) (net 8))
 (segment (start 235.082 36.94) (end 235.082 43.036) (width 0.5) (layer F.Cu) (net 8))
 (segment (start 235.082 43.036) (end 235.8046 43.7586) (width 0.5) (layer F.Cu) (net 8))
 (segment (start 235.8046 43.7586) (end 238.2311 43.7586) (width 0.5) (layer F.Cu) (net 8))
 (segment (start 238.2311 43.7586) (end 238.2311 46.1851) (width 0.25) (layer F.Cu) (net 8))
 (segment (start 256.266 48.014) (end 257.166 48.014) (width 0.5) (layer F.Cu) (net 8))
 (segment (start 254.64 49.64) (end 256.266 48.014) (width 0.5) (layer F.Cu) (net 8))
 (segment (start 253.37 49.64) (end 254.64 49.64) (width 0.5) (layer F.Cu) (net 8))
 (via (at 253.37 49.64) (size 1.2) (drill 0.8) (layers F.Cu B.Cu) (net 8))
 (via (at 240.416 48.37) (size 1.2) (drill 0.8) (layers F.Cu B.Cu) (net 8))
 (segment (start 238.2311 46.1851) (end 240.416 48.37) (width 0.5) (layer F.Cu) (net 8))
 (segment (start 238.2311 43.7586) (end 238.2311 49.7411) (width 0.5) (layer F.Cu) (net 8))
 (segment (start 241.3436 52.8536) (end 247.3261 52.8536) (width 0.5) (layer F.Cu) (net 8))
 (segment (start 238.2311 49.7411) (end 241.3436 52.8536) (width 0.5) (layer F.Cu) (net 8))
 (segment (start 250.66 34.04) (end 250.65 34.04) (width 0.5) (layer F.Cu) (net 9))
 (segment (start 250.66 34.04) (end 249.2311 32.6111) (width 0.5) (layer F.Cu) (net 9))
 (segment (start 249.2311 30.8536) (end 249.2311 32.6111) (width 0.5) (layer F.Cu) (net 9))
 (segment (start 250.962 36.178) (end 249.56 36.178) (width 0.5) (layer F.Cu) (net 9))
 (segment (start 251.5 35.64) (end 250.962 36.178) (width 0.5) (layer F.Cu) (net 9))
 (segment (start 251.5 34.89) (end 251.5 35.64) (width 0.5) (layer F.Cu) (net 9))
 (segment (start 250.65 34.04) (end 251.5 34.89) (width 0.5) (layer F.Cu) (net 9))
 (segment (start 243.845 36.178) (end 249.56 36.178) (width 0.5) (layer F.Cu) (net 9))
 (segment (start 249.2311 32.0391) (end 249.2311 30.8536) (width 0.25) (layer F.Cu) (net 9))
 (segment (start 246.004 34.908) (end 242.702 31.606) (width 0.25) (layer B.Cu) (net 10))
 (segment (start 242.702 31.606) (end 242.702 29.066) (width 0.25) (layer B.Cu) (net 10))
 (segment (start 242.702 29.066) (end 244.48 27.288) (width 0.25) (layer B.Cu) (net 10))
 (segment (start 244.48 27.288) (end 249.306 27.288) (width 0.25) (layer B.Cu) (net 10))
 (segment (start 249.306 27.288) (end 253.116 31.098) (width 0.25) (layer B.Cu) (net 10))
 (segment (start 253.116 31.098) (end 253.116 34.908) (width 0.25) (layer B.Cu) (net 10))
 (segment (start 253.116 34.908) (end 257.18 38.972) (width 0.25) (layer B.Cu) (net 10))
 (segment (start 243.845 33.638) (end 244.734 33.638) (width 0.25) (layer F.Cu) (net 10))
 (segment (start 244.734 33.638) (end 246.004 34.908) (width 0.5) (layer F.Cu) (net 10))
 (via (at 246.004 34.908) (size 1.2) (drill 0.8) (layers F.Cu B.Cu) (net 10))
 (via (at 257.18 38.972) (size 1.2) (drill 0.8) (layers F.Cu B.Cu) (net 10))
 (segment (start 257.18 38.972) (end 257.688 39.48) (width 0.5) (layer F.Cu) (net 10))
 (segment (start 257.688 39.48) (end 257.688 41.004) (width 0.5) (layer F.Cu) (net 10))
 (segment (start 257.688 41.004) (end 258.5376 41.8536) (width 0.5) (layer F.Cu) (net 10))
 (segment (start 258.5376 41.8536) (end 260.6061 41.8536) (width 0.5) (layer F.Cu) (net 10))
 (segment (start 259.5536 41.8536) (end 260.6061 41.8536) (width 0.25) (layer F.Cu) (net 10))
 (segment (start 240.67 51.164) (end 243.464 51.164) (width 0.25) (layer B.Cu) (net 11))
 (segment (start 238.13 48.624) (end 240.67 51.164) (width 0.25) (layer B.Cu) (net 11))
 (segment (start 238.13 41.512) (end 238.13 48.624) (width 0.25) (layer B.Cu) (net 11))
 (segment (start 240.162 39.48) (end 238.13 41.512) (width 0.25) (layer B.Cu) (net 11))
 (segment (start 242.702 39.48) (end 240.162 39.48) (width 0.25) (layer B.Cu) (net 11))
 (segment (start 243.21 38.972) (end 242.702 39.48) (width 0.25) (layer B.Cu) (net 11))
 (segment (start 243.845 31.098) (end 241.94 31.098) (width 0.5) (layer F.Cu) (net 11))
 (segment (start 249.2311 50.5811) (end 249.2311 52.8536) (width 0.5) (layer F.Cu) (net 11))
 (segment (start 247.909 49.259) (end 249.2311 50.5811) (width 0.5) (layer F.Cu) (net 11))
 (segment (start 245.369 49.259) (end 247.909 49.259) (width 0.5) (layer F.Cu) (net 11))
 (segment (start 243.464 51.164) (end 245.369 49.259) (width 0.5) (layer F.Cu) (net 11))
 (via (at 243.464 51.164) (size 1.2) (drill 0.8) (layers F.Cu B.Cu) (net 11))
 (via (at 243.21 38.972) (size 1.2) (drill 0.8) (layers F.Cu B.Cu) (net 11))
 (segment (start 243.21 39.08) (end 243.21 38.972) (width 0.5) (layer F.Cu) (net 11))
 (segment (start 240.68 36.55) (end 243.21 39.08) (width 0.5) (layer F.Cu) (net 11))
 (segment (start 240.68 32.358) (end 240.68 36.55) (width 0.5) (layer F.Cu) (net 11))
 (segment (start 241.94 31.098) (end 240.68 32.358) (width 0.5) (layer F.Cu) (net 11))
 (segment (start 238.2311 41.8536) (end 239.8204 41.8536) (width 0.5) (layer F.Cu) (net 12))
 (segment (start 237.876 29.828) (end 235.971 29.828) (width 0.5) (layer F.Cu) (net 12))
 (segment (start 238.384 30.336) (end 237.876 29.828) (width 0.5) (layer F.Cu) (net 12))
 (segment (start 238.384 36.934) (end 238.384 30.336) (width 0.5) (layer F.Cu) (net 12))
 (segment (start 240.416 38.966) (end 238.384 36.934) (width 0.5) (layer F.Cu) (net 12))
 (segment (start 240.416 41.258) (end 240.416 38.966) (width 0.5) (layer F.Cu) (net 12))
 (segment (start 239.8204 41.8536) (end 240.416 41.258) (width 0.5) (layer F.Cu) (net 12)))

